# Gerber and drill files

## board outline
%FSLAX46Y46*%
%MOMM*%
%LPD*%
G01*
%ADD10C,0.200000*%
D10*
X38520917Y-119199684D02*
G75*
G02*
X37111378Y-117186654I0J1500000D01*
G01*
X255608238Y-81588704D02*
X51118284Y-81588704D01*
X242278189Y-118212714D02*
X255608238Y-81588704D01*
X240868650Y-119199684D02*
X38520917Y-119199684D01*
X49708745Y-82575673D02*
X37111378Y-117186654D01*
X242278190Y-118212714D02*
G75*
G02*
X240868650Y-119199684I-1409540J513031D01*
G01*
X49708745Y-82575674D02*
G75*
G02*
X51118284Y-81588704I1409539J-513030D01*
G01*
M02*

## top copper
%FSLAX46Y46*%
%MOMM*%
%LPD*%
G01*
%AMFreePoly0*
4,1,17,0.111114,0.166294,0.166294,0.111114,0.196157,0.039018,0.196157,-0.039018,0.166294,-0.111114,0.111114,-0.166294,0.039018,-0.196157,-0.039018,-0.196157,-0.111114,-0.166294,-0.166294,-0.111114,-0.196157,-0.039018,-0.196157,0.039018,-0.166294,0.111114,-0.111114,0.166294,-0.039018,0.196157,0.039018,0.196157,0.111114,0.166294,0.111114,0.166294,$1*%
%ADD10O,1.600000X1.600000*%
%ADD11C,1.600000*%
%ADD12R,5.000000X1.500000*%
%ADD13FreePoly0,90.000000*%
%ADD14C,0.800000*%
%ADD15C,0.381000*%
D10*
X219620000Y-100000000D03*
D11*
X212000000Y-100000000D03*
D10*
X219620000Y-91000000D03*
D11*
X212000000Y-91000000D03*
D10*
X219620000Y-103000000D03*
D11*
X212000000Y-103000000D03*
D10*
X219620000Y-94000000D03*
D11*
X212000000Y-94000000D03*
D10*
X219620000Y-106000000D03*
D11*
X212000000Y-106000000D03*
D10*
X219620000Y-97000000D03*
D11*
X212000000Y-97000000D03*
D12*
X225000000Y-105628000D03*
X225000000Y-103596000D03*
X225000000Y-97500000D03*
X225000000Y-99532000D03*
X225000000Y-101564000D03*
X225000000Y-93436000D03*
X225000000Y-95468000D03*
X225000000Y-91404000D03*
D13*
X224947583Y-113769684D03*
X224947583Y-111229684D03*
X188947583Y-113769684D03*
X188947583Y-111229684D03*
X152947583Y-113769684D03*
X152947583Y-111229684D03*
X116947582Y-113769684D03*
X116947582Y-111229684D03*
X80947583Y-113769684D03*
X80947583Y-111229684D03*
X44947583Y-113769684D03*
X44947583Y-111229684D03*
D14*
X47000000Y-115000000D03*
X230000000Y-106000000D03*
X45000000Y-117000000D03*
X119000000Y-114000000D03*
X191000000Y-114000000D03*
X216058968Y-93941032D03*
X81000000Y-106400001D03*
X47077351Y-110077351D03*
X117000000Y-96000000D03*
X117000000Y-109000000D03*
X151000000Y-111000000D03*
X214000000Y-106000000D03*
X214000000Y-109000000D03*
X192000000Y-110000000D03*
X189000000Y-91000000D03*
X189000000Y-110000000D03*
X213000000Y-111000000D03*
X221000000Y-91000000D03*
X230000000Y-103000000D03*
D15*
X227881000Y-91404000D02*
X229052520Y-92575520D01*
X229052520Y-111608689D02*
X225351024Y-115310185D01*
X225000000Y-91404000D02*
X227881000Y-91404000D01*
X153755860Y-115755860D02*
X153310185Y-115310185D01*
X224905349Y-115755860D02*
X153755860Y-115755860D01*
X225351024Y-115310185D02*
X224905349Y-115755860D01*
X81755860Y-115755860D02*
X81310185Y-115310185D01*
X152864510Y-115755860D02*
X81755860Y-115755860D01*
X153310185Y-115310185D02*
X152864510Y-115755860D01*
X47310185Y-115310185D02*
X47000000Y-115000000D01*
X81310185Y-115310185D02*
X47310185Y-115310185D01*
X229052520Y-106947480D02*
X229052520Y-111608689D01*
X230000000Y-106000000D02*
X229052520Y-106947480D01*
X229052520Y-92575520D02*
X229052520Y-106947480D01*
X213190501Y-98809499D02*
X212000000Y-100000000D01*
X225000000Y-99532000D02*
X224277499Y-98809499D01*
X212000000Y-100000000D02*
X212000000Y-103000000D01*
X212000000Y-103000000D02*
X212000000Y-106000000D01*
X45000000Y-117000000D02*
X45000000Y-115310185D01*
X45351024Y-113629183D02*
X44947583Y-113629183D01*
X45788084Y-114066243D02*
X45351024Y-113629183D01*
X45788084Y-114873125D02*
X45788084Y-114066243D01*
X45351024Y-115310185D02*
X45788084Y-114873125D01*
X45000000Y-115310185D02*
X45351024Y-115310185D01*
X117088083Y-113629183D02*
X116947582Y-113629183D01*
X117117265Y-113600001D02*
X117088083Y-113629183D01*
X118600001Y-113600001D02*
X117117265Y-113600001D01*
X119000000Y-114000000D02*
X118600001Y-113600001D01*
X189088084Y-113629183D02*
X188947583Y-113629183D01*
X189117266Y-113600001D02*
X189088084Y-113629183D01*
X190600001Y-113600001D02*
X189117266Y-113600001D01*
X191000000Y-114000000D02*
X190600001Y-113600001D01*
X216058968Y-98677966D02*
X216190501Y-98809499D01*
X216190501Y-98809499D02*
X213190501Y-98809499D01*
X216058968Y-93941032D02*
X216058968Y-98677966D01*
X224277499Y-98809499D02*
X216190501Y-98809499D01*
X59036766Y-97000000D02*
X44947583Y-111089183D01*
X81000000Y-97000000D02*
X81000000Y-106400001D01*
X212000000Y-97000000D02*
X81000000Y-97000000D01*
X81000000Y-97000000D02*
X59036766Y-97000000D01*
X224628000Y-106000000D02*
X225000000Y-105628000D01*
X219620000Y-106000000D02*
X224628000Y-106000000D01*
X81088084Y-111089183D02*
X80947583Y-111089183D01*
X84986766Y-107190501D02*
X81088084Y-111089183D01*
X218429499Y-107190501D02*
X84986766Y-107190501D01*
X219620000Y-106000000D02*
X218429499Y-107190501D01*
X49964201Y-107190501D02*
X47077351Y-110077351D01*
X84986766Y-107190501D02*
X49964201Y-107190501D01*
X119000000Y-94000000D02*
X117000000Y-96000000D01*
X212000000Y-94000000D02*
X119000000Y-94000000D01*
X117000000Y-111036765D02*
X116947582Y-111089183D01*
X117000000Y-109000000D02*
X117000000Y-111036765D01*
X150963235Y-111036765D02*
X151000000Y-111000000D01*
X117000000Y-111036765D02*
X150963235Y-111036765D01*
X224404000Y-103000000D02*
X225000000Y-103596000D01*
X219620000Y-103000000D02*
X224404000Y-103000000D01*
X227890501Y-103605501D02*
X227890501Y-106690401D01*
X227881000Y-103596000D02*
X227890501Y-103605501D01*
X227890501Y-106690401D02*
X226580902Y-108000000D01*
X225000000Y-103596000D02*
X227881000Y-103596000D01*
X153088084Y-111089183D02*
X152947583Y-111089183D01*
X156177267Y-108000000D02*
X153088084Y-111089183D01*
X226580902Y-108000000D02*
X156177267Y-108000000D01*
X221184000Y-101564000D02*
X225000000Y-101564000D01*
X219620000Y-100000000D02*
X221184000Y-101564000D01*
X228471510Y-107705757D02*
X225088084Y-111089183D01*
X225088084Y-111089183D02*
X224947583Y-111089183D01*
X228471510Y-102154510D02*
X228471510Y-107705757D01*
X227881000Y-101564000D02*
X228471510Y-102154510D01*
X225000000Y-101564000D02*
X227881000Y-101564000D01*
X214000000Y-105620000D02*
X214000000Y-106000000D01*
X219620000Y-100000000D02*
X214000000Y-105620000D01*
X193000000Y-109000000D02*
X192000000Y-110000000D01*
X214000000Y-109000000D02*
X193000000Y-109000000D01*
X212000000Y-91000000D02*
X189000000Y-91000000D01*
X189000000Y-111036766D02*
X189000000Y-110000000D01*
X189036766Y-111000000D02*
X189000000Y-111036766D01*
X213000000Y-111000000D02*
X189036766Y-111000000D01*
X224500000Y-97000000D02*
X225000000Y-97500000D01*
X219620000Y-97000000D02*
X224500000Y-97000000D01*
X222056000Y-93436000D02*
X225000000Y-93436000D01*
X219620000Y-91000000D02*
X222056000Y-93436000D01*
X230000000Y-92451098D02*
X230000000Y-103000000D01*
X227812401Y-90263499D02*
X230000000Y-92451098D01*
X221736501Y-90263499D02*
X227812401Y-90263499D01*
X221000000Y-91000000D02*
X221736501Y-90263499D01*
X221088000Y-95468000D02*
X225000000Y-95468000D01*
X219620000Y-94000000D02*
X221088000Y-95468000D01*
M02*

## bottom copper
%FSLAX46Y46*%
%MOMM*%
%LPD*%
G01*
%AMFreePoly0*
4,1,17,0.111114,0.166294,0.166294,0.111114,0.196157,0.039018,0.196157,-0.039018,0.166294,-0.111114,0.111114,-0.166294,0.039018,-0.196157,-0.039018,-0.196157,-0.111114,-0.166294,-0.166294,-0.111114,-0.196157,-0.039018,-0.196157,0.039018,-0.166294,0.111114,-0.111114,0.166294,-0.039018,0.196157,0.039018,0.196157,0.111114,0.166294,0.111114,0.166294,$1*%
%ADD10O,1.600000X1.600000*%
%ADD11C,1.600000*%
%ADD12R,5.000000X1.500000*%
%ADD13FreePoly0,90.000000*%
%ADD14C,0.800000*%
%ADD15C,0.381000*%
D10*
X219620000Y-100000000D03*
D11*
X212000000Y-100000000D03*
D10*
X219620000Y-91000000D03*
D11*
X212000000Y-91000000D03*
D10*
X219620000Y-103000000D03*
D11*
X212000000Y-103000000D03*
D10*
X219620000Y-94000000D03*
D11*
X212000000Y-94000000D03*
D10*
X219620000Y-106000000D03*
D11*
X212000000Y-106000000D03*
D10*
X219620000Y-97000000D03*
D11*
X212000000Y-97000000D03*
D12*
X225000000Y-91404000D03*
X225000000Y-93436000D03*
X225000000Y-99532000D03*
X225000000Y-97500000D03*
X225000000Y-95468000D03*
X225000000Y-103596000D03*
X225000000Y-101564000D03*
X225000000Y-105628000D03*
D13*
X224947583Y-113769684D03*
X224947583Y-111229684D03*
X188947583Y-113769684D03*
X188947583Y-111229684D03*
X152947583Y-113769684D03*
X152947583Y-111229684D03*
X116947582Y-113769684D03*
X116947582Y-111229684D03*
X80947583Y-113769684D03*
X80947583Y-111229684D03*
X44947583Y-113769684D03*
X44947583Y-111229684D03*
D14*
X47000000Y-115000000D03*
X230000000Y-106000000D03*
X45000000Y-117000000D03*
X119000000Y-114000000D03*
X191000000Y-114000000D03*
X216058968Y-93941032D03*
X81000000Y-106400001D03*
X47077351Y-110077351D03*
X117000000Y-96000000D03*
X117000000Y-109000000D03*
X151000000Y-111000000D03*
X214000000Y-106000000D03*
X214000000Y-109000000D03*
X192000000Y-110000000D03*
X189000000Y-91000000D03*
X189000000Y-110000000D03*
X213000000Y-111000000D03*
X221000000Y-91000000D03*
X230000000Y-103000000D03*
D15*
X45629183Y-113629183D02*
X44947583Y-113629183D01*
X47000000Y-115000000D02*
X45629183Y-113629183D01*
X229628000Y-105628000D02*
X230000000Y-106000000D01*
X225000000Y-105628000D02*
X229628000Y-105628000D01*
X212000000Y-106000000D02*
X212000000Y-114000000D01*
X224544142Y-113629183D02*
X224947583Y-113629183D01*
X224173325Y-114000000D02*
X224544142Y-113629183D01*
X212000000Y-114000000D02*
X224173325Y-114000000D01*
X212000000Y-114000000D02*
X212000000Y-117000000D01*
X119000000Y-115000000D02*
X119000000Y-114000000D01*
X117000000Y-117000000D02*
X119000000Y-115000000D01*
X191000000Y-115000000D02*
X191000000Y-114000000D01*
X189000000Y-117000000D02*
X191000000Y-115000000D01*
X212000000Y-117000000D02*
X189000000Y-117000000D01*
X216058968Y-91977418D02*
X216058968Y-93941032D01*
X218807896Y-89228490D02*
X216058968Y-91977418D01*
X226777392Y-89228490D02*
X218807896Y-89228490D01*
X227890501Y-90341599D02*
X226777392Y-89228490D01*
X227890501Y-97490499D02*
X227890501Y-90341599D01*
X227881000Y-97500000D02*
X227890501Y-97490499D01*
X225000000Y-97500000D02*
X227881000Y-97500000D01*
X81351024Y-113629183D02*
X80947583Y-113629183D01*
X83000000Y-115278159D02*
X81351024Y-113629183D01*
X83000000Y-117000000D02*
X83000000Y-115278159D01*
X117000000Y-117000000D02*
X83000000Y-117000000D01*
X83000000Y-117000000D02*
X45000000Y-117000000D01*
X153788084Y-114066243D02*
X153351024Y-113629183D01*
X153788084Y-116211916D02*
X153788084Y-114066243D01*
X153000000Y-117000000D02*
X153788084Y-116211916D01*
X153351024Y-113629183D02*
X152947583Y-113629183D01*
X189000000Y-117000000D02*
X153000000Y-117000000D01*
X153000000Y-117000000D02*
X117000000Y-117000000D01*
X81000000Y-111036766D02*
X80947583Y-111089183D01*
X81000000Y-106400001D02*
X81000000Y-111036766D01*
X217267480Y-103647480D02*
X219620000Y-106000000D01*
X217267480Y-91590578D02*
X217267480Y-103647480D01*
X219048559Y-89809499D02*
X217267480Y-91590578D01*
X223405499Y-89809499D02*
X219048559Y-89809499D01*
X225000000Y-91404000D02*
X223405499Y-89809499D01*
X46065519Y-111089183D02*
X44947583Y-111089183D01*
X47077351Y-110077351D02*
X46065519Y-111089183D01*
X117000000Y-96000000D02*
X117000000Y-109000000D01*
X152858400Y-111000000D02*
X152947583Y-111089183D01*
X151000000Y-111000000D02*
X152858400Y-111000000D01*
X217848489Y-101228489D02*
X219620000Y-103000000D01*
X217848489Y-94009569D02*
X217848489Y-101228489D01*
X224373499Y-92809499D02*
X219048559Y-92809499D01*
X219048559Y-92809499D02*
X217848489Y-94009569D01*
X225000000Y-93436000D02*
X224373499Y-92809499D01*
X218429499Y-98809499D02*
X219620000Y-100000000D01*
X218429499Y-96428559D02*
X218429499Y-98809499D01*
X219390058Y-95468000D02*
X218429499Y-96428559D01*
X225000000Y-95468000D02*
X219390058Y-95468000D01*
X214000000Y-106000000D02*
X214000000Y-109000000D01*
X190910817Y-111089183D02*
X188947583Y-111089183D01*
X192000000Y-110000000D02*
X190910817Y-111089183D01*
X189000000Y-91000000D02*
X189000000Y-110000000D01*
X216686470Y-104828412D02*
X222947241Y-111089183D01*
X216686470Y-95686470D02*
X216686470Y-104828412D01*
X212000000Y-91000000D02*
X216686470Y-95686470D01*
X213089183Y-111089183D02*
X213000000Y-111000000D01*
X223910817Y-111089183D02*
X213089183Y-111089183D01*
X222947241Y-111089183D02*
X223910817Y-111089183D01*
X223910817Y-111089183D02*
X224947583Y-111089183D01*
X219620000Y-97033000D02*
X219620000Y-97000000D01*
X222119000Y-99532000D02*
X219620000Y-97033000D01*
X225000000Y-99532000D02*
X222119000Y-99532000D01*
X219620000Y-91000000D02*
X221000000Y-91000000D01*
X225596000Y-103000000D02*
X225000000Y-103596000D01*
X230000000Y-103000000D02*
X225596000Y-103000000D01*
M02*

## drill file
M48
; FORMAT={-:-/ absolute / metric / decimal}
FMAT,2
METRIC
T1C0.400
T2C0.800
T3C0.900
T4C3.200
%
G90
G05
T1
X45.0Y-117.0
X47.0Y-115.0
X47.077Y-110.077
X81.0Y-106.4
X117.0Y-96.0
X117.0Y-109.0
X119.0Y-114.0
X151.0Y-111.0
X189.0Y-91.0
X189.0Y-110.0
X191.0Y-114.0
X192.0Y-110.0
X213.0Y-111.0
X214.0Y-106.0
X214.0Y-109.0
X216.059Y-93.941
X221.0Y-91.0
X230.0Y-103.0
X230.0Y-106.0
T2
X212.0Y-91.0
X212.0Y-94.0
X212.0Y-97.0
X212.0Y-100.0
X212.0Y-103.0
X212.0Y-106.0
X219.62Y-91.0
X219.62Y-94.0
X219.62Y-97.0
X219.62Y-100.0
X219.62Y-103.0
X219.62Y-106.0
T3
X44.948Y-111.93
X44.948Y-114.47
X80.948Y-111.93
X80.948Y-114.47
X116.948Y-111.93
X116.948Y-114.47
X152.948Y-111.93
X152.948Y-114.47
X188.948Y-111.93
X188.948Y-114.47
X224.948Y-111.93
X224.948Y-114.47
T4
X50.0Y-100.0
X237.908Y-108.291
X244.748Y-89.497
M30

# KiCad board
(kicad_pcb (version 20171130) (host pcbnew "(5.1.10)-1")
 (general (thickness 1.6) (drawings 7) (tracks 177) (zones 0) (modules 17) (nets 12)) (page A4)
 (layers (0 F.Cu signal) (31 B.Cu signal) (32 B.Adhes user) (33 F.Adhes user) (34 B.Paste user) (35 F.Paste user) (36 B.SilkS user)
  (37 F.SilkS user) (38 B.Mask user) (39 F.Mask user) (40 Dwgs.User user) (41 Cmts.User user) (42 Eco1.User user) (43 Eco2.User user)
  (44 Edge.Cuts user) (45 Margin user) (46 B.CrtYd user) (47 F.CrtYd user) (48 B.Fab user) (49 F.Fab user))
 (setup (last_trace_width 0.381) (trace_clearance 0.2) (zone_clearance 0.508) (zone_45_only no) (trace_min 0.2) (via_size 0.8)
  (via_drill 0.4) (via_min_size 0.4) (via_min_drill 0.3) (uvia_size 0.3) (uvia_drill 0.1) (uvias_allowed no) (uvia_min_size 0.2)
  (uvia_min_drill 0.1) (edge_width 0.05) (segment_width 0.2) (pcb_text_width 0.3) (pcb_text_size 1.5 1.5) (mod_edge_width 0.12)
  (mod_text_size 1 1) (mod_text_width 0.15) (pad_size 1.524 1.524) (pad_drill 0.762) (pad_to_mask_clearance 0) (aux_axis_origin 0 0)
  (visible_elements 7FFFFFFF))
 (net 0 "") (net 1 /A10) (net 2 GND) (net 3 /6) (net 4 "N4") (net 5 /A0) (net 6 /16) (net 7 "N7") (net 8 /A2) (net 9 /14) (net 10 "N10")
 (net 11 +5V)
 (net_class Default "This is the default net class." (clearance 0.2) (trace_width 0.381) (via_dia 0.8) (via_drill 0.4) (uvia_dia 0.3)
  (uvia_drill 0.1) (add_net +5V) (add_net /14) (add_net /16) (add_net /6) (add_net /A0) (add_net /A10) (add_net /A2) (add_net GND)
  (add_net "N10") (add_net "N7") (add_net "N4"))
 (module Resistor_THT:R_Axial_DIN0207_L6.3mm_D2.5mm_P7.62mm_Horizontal (layer F.Cu) (at 212 100)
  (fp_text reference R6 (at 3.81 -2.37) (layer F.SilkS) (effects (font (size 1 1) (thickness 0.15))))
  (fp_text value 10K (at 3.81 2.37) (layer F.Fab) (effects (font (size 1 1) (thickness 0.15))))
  (pad 2 thru_hole oval (at 7.62 0) (size 1.6 1.6) (drill 0.8) (layers *.Cu *.Mask) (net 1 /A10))
  (pad 1 thru_hole circle (at 0 0) (size 1.6 1.6) (drill 0.8) (layers *.Cu *.Mask) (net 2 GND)))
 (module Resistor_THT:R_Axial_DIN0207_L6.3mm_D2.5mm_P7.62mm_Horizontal (layer F.Cu) (at 212 91)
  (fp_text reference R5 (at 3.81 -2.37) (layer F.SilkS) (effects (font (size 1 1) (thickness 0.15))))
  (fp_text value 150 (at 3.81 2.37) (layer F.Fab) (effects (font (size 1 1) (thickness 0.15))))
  (pad 2 thru_hole oval (at 7.62 0) (size 1.6 1.6) (drill 0.8) (layers *.Cu *.Mask) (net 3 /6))
  (pad 1 thru_hole circle (at 0 0) (size 1.6 1.6) (drill 0.8) (layers *.Cu *.Mask) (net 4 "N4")))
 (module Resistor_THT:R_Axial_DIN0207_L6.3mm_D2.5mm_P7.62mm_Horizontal (layer F.Cu) (at 212 103)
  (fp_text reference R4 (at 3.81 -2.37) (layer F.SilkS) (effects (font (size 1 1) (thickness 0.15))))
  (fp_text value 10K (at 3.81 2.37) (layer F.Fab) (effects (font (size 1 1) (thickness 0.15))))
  (pad 2 thru_hole oval (at 7.62 0) (size 1.6 1.6) (drill 0.8) (layers *.Cu *.Mask) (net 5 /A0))
  (pad 1 thru_hole circle (at 0 0) (size 1.6 1.6) (drill 0.8) (layers *.Cu *.Mask) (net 2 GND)))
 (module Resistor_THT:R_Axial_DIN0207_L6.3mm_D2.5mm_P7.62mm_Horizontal (layer F.Cu) (at 212 94)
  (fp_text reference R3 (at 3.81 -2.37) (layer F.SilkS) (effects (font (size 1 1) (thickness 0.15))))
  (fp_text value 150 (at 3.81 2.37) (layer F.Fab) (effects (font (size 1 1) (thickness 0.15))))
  (pad 2 thru_hole oval (at 7.62 0) (size 1.6 1.6) (drill 0.8) (layers *.Cu *.Mask) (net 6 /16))
  (pad 1 thru_hole circle (at 0 0) (size 1.6 1.6) (drill 0.8) (layers *.Cu *.Mask) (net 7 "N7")))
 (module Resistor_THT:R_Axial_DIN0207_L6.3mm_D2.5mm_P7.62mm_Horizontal (layer F.Cu) (at 212 106)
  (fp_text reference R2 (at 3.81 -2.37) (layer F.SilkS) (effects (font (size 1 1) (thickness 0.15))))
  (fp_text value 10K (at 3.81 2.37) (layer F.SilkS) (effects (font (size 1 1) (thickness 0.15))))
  (pad 2 thru_hole oval (at 7.62 0) (size 1.6 1.6) (drill 0.8) (layers *.Cu *.Mask) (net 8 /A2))
  (pad 1 thru_hole circle (at 0 0) (size 1.6 1.6) (drill 0.8) (layers *.Cu *.Mask) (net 2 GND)))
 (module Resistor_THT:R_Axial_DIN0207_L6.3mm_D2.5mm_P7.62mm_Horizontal (layer F.Cu) (at 212 97)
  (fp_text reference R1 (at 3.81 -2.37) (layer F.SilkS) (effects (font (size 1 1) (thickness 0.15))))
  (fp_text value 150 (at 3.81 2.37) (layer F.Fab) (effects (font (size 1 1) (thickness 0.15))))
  (pad 2 thru_hole oval (at 7.62 0) (size 1.6 1.6) (drill 0.8) (layers *.Cu *.Mask) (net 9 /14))
  (pad 1 thru_hole circle (at 0 0) (size 1.6 1.6) (drill 0.8) (layers *.Cu *.Mask) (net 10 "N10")))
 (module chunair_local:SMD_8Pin (layer B.Cu) (at 225 99.532)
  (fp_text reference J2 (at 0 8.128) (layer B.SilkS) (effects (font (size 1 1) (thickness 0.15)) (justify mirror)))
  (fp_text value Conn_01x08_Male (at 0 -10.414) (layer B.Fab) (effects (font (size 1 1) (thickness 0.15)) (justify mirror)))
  (pad 8 smd rect (at 0 -8.128) (size 5 1.5) (layers B.Cu B.Paste B.Mask) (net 8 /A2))
  (pad 7 smd rect (at 0 -6.096) (size 5 1.5) (layers B.Cu B.Paste B.Mask) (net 5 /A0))
  (pad 4 smd rect (at 0 0) (size 5 1.5) (layers B.Cu B.Paste B.Mask) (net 9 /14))
  (pad 5 smd rect (at 0 -2.032) (size 5 1.5) (layers B.Cu B.Paste B.Mask) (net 2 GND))
  (pad 6 smd rect (at 0 -4.064) (size 5 1.5) (layers B.Cu B.Paste B.Mask) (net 1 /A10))
  (pad 2 smd rect (at 0 4.064) (size 5 1.5) (layers B.Cu B.Paste B.Mask) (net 3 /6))
  (pad 3 smd rect (at 0 2.032) (size 5 1.5) (layers B.Cu B.Paste B.Mask) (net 6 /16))
  (pad 1 smd rect (at 0 6.096) (size 5 1.5) (layers B.Cu B.Paste B.Mask) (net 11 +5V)))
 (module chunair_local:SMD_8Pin (layer F.Cu) (at 225 97.5)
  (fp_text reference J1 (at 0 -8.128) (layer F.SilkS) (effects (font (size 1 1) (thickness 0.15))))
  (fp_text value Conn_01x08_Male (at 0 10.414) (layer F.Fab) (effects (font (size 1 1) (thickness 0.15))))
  (pad 8 smd rect (at 0 8.128) (size 5 1.5) (layers F.Cu F.Paste F.Mask) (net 8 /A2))
  (pad 7 smd rect (at 0 6.096) (size 5 1.5) (layers F.Cu F.Paste F.Mask) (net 5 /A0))
  (pad 4 smd rect (at 0 0) (size 5 1.5) (layers F.Cu F.Paste F.Mask) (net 9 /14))
  (pad 5 smd rect (at 0 2.032) (size 5 1.5) (layers F.Cu F.Paste F.Mask) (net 2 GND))
  (pad 6 smd rect (at 0 4.064) (size 5 1.5) (layers F.Cu F.Paste F.Mask) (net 1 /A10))
  (pad 2 smd rect (at 0 -4.064) (size 5 1.5) (layers F.Cu F.Paste F.Mask) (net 3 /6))
  (pad 3 smd rect (at 0 -2.032) (size 5 1.5) (layers F.Cu F.Paste F.Mask) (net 6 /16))
  (pad 1 smd rect (at 0 -6.096) (size 5 1.5) (layers F.Cu F.Paste F.Mask) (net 11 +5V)))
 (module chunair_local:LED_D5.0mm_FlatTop (layer F.Cu) (at 224.947583 114.469684 90)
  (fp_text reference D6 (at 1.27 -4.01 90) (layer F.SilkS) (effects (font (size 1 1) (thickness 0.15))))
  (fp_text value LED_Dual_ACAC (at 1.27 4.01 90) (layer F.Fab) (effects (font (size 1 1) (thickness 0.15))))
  (pad 2 smd custom (at 0.7 0 90) (size 0.4 0.4) (layers F.Cu F.Mask) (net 11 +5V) (zone_connect 0)
   (options (clearance outline) (anchor circle)) (primitives))
  (pad 4 smd custom (at 0.7 0 90) (size 0.4 0.4) (layers B.Cu B.Mask) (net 2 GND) (zone_connect 0)
   (options (clearance outline) (anchor circle)) (primitives))
  (pad 1 smd custom (at 3.24 0 90) (size 0.4 0.4) (layers F.Cu F.Mask) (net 1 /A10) (options (clearance outline) (anchor circle))
   (primitives))
  (pad 3 smd custom (at 3.24 0 90) (size 0.4 0.4) (layers B.Cu B.Mask) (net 4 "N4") (zone_connect 0)
   (options (clearance outline) (anchor circle)) (primitives))
  (pad "" np_thru_hole circle (at 2.54 0 90) (size 0.9 0.9) (drill 0.9) (layers *.Cu *.Mask))
  (pad "" np_thru_hole circle (at 0 0 90) (size 0.9 0.9) (drill 0.9) (layers *.Cu *.Mask)))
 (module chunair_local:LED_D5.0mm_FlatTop (layer F.Cu) (at 188.947583 114.469684 90)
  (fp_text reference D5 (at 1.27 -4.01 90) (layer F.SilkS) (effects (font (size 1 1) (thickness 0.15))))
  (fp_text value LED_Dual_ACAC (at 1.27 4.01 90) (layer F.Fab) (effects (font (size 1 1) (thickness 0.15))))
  (pad 2 smd custom (at 0.7 0 90) (size 0.4 0.4) (layers F.Cu F.Mask) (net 2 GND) (zone_connect 0)
   (options (clearance outline) (anchor circle)) (primitives))
  (pad 4 smd custom (at 0.7 0 90) (size 0.4 0.4) (layers B.Cu B.Mask) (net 11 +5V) (zone_connect 0)
   (options (clearance outline) (anchor circle)) (primitives))
  (pad 1 smd custom (at 3.24 0 90) (size 0.4 0.4) (layers F.Cu F.Mask) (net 4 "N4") (options (clearance outline) (anchor circle))
   (primitives))
  (pad 3 smd custom (at 3.24 0 90) (size 0.4 0.4) (layers B.Cu B.Mask) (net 1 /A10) (zone_connect 0)
   (options (clearance outline) (anchor circle)) (primitives))
  (pad "" np_thru_hole circle (at 2.54 0 90) (size 0.9 0.9) (drill 0.9) (layers *.Cu *.Mask))
  (pad "" np_thru_hole circle (at 0 0 90) (size 0.9 0.9) (drill 0.9) (layers *.Cu *.Mask)))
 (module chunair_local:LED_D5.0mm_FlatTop (layer F.Cu) (at 152.947583 114.469684 90)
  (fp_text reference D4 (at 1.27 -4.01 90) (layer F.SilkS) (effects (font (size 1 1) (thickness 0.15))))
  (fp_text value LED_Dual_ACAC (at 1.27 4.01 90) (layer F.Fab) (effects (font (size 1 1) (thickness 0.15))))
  (pad 2 smd custom (at 0.7 0 90) (size 0.4 0.4) (layers F.Cu F.Mask) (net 11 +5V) (zone_connect 0)
   (options (clearance outline) (anchor circle)) (primitives))
  (pad 4 smd custom (at 0.7 0 90) (size 0.4 0.4) (layers B.Cu B.Mask) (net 2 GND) (zone_connect 0)
   (options (clearance outline) (anchor circle)) (primitives))
  (pad 1 smd custom (at 3.24 0 90) (size 0.4 0.4) (layers F.Cu F.Mask) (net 5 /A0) (options (clearance outline) (anchor circle))
   (primitives))
  (pad 3 smd custom (at 3.24 0 90) (size 0.4 0.4) (layers B.Cu B.Mask) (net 7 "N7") (zone_connect 0)
   (options (clearance outline) (anchor circle)) (primitives))
  (pad "" np_thru_hole circle (at 2.54 0 90) (size 0.9 0.9) (drill 0.9) (layers *.Cu *.Mask))
  (pad "" np_thru_hole circle (at 0 0 90) (size 0.9 0.9) (drill 0.9) (layers *.Cu *.Mask)))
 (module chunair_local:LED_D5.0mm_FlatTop (layer F.Cu) (at 116.947582 114.469684 90)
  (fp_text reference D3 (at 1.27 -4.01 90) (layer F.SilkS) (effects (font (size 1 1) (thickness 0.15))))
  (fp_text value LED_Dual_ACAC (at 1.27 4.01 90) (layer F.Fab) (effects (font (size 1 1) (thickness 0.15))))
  (pad 2 smd custom (at 0.7 0 90) (size 0.4 0.4) (layers F.Cu F.Mask) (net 2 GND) (zone_connect 0)
   (options (clearance outline) (anchor circle)) (primitives))
  (pad 4 smd custom (at 0.7 0 90) (size 0.4 0.4) (layers B.Cu B.Mask) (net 11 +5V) (zone_connect 0)
   (options (clearance outline) (anchor circle)) (primitives))
  (pad 1 smd custom (at 3.24 0 90) (size 0.4 0.4) (layers F.Cu F.Mask) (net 7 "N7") (options (clearance outline) (anchor circle))
   (primitives))
  (pad 3 smd custom (at 3.24 0 90) (size 0.4 0.4) (layers B.Cu B.Mask) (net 5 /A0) (zone_connect 0)
   (options (clearance outline) (anchor circle)) (primitives))
  (pad "" np_thru_hole circle (at 2.54 0 90) (size 0.9 0.9) (drill 0.9) (layers *.Cu *.Mask))
  (pad "" np_thru_hole circle (at 0 0 90) (size 0.9 0.9) (drill 0.9) (layers *.Cu *.Mask)))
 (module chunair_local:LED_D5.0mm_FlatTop (layer F.Cu) (at 80.947583 114.469684 90)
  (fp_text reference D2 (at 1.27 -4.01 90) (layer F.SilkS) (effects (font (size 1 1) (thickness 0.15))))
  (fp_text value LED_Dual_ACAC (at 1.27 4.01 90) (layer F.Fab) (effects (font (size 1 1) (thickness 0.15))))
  (pad 2 smd custom (at 0.7 0 90) (size 0.4 0.4) (layers F.Cu F.Mask) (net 11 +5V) (zone_connect 0)
   (options (clearance outline) (anchor circle)) (primitives))
  (pad 4 smd custom (at 0.7 0 90) (size 0.4 0.4) (layers B.Cu B.Mask) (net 2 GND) (zone_connect 0)
   (options (clearance outline) (anchor circle)) (primitives))
  (pad 1 smd custom (at 3.24 0 90) (size 0.4 0.4) (layers F.Cu F.Mask) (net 8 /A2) (options (clearance outline) (anchor circle))
   (primitives))
  (pad 3 smd custom (at 3.24 0 90) (size 0.4 0.4) (layers B.Cu B.Mask) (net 10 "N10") (zone_connect 0)
   (options (clearance outline) (anchor circle)) (primitives))
  (pad "" np_thru_hole circle (at 2.54 0 90) (size 0.9 0.9) (drill 0.9) (layers *.Cu *.Mask))
  (pad "" np_thru_hole circle (at 0 0 90) (size 0.9 0.9) (drill 0.9) (layers *.Cu *.Mask)))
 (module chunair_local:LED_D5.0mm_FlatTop (layer F.Cu) (at 44.947583 114.469684 90)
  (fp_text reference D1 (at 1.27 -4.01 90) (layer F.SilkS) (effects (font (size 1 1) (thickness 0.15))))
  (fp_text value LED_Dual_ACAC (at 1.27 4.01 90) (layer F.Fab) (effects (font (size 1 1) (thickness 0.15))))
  (pad 2 smd custom (at 0.7 0 90) (size 0.4 0.4) (layers F.Cu F.Mask) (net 2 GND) (zone_connect 0)
   (options (clearance outline) (anchor circle)) (primitives))
  (pad 4 smd custom (at 0.7 0 90) (size 0.4 0.4) (layers B.Cu B.Mask) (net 11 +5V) (zone_connect 0)
   (options (clearance outline) (anchor circle)) (primitives))
  (pad 1 smd custom (at 3.24 0 90) (size 0.4 0.4) (layers F.Cu F.Mask) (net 10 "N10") (options (clearance outline) (anchor circle))
   (primitives))
  (pad 3 smd custom (at 3.24 0 90) (size 0.4 0.4) (layers B.Cu B.Mask) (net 8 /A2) (zone_connect 0)
   (options (clearance outline) (anchor circle)) (primitives))
  (pad "" np_thru_hole circle (at 2.54 0 90) (size 0.9 0.9) (drill 0.9) (layers *.Cu *.Mask))
  (pad "" np_thru_hole circle (at 0 0 90) (size 0.9 0.9) (drill 0.9) (layers *.Cu *.Mask)))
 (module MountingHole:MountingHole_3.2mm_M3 (layer F.Cu) (at 244.748423 89.497267)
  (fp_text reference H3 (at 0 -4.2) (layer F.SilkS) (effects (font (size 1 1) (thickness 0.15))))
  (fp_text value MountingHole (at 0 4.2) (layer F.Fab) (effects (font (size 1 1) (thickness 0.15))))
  (pad 1 np_thru_hole circle (at 0 0) (size 3.2 3.2) (drill 3.2) (layers *.Cu *.Mask)))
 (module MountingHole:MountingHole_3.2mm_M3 (layer F.Cu) (at 237.90802 108.29112)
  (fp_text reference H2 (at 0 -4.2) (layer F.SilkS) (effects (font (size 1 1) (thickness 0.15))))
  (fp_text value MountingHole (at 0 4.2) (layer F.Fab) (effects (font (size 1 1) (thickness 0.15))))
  (pad 1 np_thru_hole circle (at 0 0) (size 3.2 3.2) (drill 3.2) (layers *.Cu *.Mask)))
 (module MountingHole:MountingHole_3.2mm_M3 (layer F.Cu) (at 50 100)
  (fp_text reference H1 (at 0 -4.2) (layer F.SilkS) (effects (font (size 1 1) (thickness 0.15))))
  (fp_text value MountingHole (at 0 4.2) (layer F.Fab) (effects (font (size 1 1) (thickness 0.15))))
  (pad 1 np_thru_hole circle (at 0 0) (size 3.2 3.2) (drill 3.2) (layers *.Cu *.Mask)))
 (gr_arc (start 38.520917 117.699684) (end 37.111378 117.186654) (angle -110) (layer Edge.Cuts) (width 0.2))
 (gr_line (start 255.608238 81.588704) (end 51.118284 81.588704) (layer Edge.Cuts) (width 0.2))
 (gr_line (start 242.278189 118.212714) (end 255.608238 81.588704) (layer Edge.Cuts) (width 0.2))
 (gr_line (start 240.86865 119.199684) (end 38.520917 119.199684) (layer Edge.Cuts) (width 0.2))
 (gr_line (start 49.708745 82.575673) (end 37.111378 117.186654) (layer Edge.Cuts) (width 0.2))
 (gr_arc (start 240.86865 117.699683) (end 240.86865 119.199684) (angle -70) (layer Edge.Cuts) (width 0.2))
 (gr_arc (start 51.118284 83.088704) (end 51.118284 81.588704) (angle -70) (layer Edge.Cuts) (width 0.2))
 (segment (start 227.881 91.404) (end 229.05252 92.57552) (width 0.381) (layer F.Cu) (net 11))
 (segment (start 229.05252 111.608689) (end 225.351024 115.310185) (width 0.381) (layer F.Cu) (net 11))
 (segment (start 225 91.404) (end 227.881 91.404) (width 0.381) (layer F.Cu) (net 11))
 (segment (start 153.75586 115.75586) (end 153.310185 115.310185) (width 0.381) (layer F.Cu) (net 11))
 (segment (start 224.905349 115.75586) (end 153.75586 115.75586) (width 0.381) (layer F.Cu) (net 11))
 (segment (start 225.351024 115.310185) (end 224.905349 115.75586) (width 0.381) (layer F.Cu) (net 11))
 (segment (start 81.75586 115.75586) (end 81.310185 115.310185) (width 0.381) (layer F.Cu) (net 11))
 (segment (start 152.86451 115.75586) (end 81.75586 115.75586) (width 0.381) (layer F.Cu) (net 11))
 (segment (start 153.310185 115.310185) (end 152.86451 115.75586) (width 0.381) (layer F.Cu) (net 11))
 (via (at 47 115) (size 0.8) (drill 0.4) (layers F.Cu B.Cu) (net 11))
 (segment (start 47.310185 115.310185) (end 47 115) (width 0.381) (layer F.Cu) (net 11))
 (segment (start 81.310185 115.310185) (end 47.310185 115.310185) (width 0.381) (layer F.Cu) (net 11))
 (segment (start 45.629183 113.629183) (end 44.947583 113.629183) (width 0.381) (layer B.Cu) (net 11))
 (segment (start 47 115) (end 45.629183 113.629183) (width 0.381) (layer B.Cu) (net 11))
 (via (at 230 106) (size 0.8) (drill 0.4) (layers F.Cu B.Cu) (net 11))
 (segment (start 229.628 105.628) (end 230 106) (width 0.381) (layer B.Cu) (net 11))
 (segment (start 225 105.628) (end 229.628 105.628) (width 0.381) (layer B.Cu) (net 11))
 (segment (start 229.05252 106.94748) (end 229.05252 111.608689) (width 0.381) (layer F.Cu) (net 11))
 (segment (start 230 106) (end 229.05252 106.94748) (width 0.381) (layer F.Cu) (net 11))
 (segment (start 229.05252 92.57552) (end 229.05252 106.94748) (width 0.381) (layer F.Cu) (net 11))
 (segment (start 213.190501 98.809499) (end 212 100) (width 0.381) (layer F.Cu) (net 2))
 (segment (start 225 99.532) (end 224.277499 98.809499) (width 0.381) (layer F.Cu) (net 2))
 (segment (start 212 100) (end 212 103) (width 0.381) (layer F.Cu) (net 2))
 (segment (start 212 103) (end 212 106) (width 0.381) (layer F.Cu) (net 2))
 (segment (start 212 106) (end 212 114) (width 0.381) (layer B.Cu) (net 2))
 (segment (start 224.544142 113.629183) (end 224.947583 113.629183) (width 0.381) (layer B.Cu) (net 2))
 (segment (start 224.173325 114) (end 224.544142 113.629183) (width 0.381) (layer B.Cu) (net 2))
 (segment (start 212 114) (end 224.173325 114) (width 0.381) (layer B.Cu) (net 2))
 (segment (start 212 114) (end 212 117) (width 0.381) (layer B.Cu) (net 2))
 (via (at 45 117) (size 0.8) (drill 0.4) (layers F.Cu B.Cu) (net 2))
 (segment (start 45 117) (end 45 115.310185) (width 0.381) (layer F.Cu) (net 2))
 (segment (start 45.351024 113.629183) (end 44.947583 113.629183) (width 0.381) (layer F.Cu) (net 2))
 (segment (start 45.788084 114.066243) (end 45.351024 113.629183) (width 0.381) (layer F.Cu) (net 2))
 (segment (start 45.788084 114.873125) (end 45.788084 114.066243) (width 0.381) (layer F.Cu) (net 2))
 (segment (start 45.351024 115.310185) (end 45.788084 114.873125) (width 0.381) (layer F.Cu) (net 2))
 (segment (start 45 115.310185) (end 45.351024 115.310185) (width 0.381) (layer F.Cu) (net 2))
 (via (at 119 114) (size 0.8) (drill 0.4) (layers F.Cu B.Cu) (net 2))
 (segment (start 119 115) (end 119 114) (width 0.381) (layer B.Cu) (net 2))
 (segment (start 117 117) (end 119 115) (width 0.381) (layer B.Cu) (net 2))
 (segment (start 117.088083 113.629183) (end 116.947582 113.629183) (width 0.381) (layer F.Cu) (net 2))
 (segment (start 117.117265 113.600001) (end 117.088083 113.629183) (width 0.381) (layer F.Cu) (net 2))
 (segment (start 118.600001 113.600001) (end 117.117265 113.600001) (width 0.381) (layer F.Cu) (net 2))
 (segment (start 119 114) (end 118.600001 113.600001) (width 0.381) (layer F.Cu) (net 2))
 (via (at 191 114) (size 0.8) (drill 0.4) (layers F.Cu B.Cu) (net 2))
 (segment (start 191 115) (end 191 114) (width 0.381) (layer B.Cu) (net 2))
 (segment (start 189 117) (end 191 115) (width 0.381) (layer B.Cu) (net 2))
 (segment (start 212 117) (end 189 117) (width 0.381) (layer B.Cu) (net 2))
 (segment (start 189.088084 113.629183) (end 188.947583 113.629183) (width 0.381) (layer F.Cu) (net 2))
 (segment (start 189.117266 113.600001) (end 189.088084 113.629183) (width 0.381) (layer F.Cu) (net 2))
 (segment (start 190.600001 113.600001) (end 189.117266 113.600001) (width 0.381) (layer F.Cu) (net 2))
 (segment (start 191 114) (end 190.600001 113.600001) (width 0.381) (layer F.Cu) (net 2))
 (segment (start 216.058968 91.977418) (end 216.058968 93.941032) (width 0.381) (layer B.Cu) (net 2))
 (via (at 216.058968 93.941032) (size 0.8) (drill 0.4) (layers F.Cu B.Cu) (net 2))
 (segment (start 218.807896 89.22849) (end 216.058968 91.977418) (width 0.381) (layer B.Cu) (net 2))
 (segment (start 226.777392 89.22849) (end 218.807896 89.22849) (width 0.381) (layer B.Cu) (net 2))
 (segment (start 227.890501 90.341599) (end 226.777392 89.22849) (width 0.381) (layer B.Cu) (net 2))
 (segment (start 227.890501 97.490499) (end 227.890501 90.341599) (width 0.381) (layer B.Cu) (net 2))
 (segment (start 227.881 97.5) (end 227.890501 97.490499) (width 0.381) (layer B.Cu) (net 2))
 (segment (start 225 97.5) (end 227.881 97.5) (width 0.381) (layer B.Cu) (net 2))
 (segment (start 216.058968 98.677966) (end 216.190501 98.809499) (width 0.381) (layer F.Cu) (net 2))
 (segment (start 216.190501 98.809499) (end 213.190501 98.809499) (width 0.381) (layer F.Cu) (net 2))
 (segment (start 216.058968 93.941032) (end 216.058968 98.677966) (width 0.381) (layer F.Cu) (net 2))
 (segment (start 224.277499 98.809499) (end 216.190501 98.809499) (width 0.381) (layer F.Cu) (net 2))
 (segment (start 81.351024 113.629183) (end 80.947583 113.629183) (width 0.381) (layer B.Cu) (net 2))
 (segment (start 83 115.278159) (end 81.351024 113.629183) (width 0.381) (layer B.Cu) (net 2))
 (segment (start 83 117) (end 83 115.278159) (width 0.381) (layer B.Cu) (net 2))
 (segment (start 117 117) (end 83 117) (width 0.381) (layer B.Cu) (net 2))
 (segment (start 83 117) (end 45 117) (width 0.381) (layer B.Cu) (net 2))
 (segment (start 153.788084 114.066243) (end 153.351024 113.629183) (width 0.381) (layer B.Cu) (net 2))
 (segment (start 153.788084 116.211916) (end 153.788084 114.066243) (width 0.381) (layer B.Cu) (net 2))
 (segment (start 153 117) (end 153.788084 116.211916) (width 0.381) (layer B.Cu) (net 2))
 (segment (start 153.351024 113.629183) (end 152.947583 113.629183) (width 0.381) (layer B.Cu) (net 2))
 (segment (start 189 117) (end 153 117) (width 0.381) (layer B.Cu) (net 2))
 (segment (start 153 117) (end 117 117) (width 0.381) (layer B.Cu) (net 2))
 (segment (start 59.036766 97) (end 44.947583 111.089183) (width 0.381) (layer F.Cu) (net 10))
 (segment (start 81 97) (end 81 106.400001) (width 0.381) (layer F.Cu) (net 10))
 (segment (start 212 97) (end 81 97) (width 0.381) (layer F.Cu) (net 10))
 (via (at 81 106.400001) (size 0.8) (drill 0.4) (layers F.Cu B.Cu) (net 10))
 (segment (start 81 97) (end 59.036766 97) (width 0.381) (layer F.Cu) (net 10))
 (segment (start 81 111.036766) (end 80.947583 111.089183) (width 0.381) (layer B.Cu) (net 10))
 (segment (start 81 106.400001) (end 81 111.036766) (width 0.381) (layer B.Cu) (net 10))
 (segment (start 224.628 106) (end 225 105.628) (width 0.381) (layer F.Cu) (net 8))
 (segment (start 219.62 106) (end 224.628 106) (width 0.381) (layer F.Cu) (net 8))
 (segment (start 81.088084 111.089183) (end 80.947583 111.089183) (width 0.381) (layer F.Cu) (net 8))
 (segment (start 84.986766 107.190501) (end 81.088084 111.089183) (width 0.381) (layer F.Cu) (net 8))
 (segment (start 218.429499 107.190501) (end 84.986766 107.190501) (width 0.381) (layer F.Cu) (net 8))
 (segment (start 219.62 106) (end 218.429499 107.190501) (width 0.381) (layer F.Cu) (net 8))
 (segment (start 217.26748 103.64748) (end 219.62 106) (width 0.381) (layer B.Cu) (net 8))
 (segment (start 217.26748 91.590578) (end 217.26748 103.64748) (width 0.381) (layer B.Cu) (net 8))
 (segment (start 219.048559 89.809499) (end 217.26748 91.590578) (width 0.381) (layer B.Cu) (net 8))
 (segment (start 223.405499 89.809499) (end 219.048559 89.809499) (width 0.381) (layer B.Cu) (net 8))
 (segment (start 225 91.404) (end 223.405499 89.809499) (width 0.381) (layer B.Cu) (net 8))
 (via (at 47.077351 110.077351) (size 0.8) (drill 0.4) (layers F.Cu B.Cu) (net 8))
 (segment (start 49.964201 107.190501) (end 47.077351 110.077351) (width 0.381) (layer F.Cu) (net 8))
 (segment (start 84.986766 107.190501) (end 49.964201 107.190501) (width 0.381) (layer F.Cu) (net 8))
 (segment (start 46.065519 111.089183) (end 44.947583 111.089183) (width 0.381) (layer B.Cu) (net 8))
 (segment (start 47.077351 110.077351) (end 46.065519 111.089183) (width 0.381) (layer B.Cu) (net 8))
 (via (at 117 96) (size 0.8) (drill 0.4) (layers F.Cu B.Cu) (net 7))
 (segment (start 119 94) (end 117 96) (width 0.381) (layer F.Cu) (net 7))
 (segment (start 212 94) (end 119 94) (width 0.381) (layer F.Cu) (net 7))
 (via (at 117 109) (size 0.8) (drill 0.4) (layers F.Cu B.Cu) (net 7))
 (segment (start 117 96) (end 117 109) (width 0.381) (layer B.Cu) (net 7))
 (segment (start 117 111.036765) (end 116.947582 111.089183) (width 0.381) (layer F.Cu) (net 7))
 (segment (start 117 109) (end 117 111.036765) (width 0.381) (layer F.Cu) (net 7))
 (via (at 151 111) (size 0.8) (drill 0.4) (layers F.Cu B.Cu) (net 7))
 (segment (start 150.963235 111.036765) (end 151 111) (width 0.381) (layer F.Cu) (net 7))
 (segment (start 117 111.036765) (end 150.963235 111.036765) (width 0.381) (layer F.Cu) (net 7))
 (segment (start 152.8584 111) (end 152.947583 111.089183) (width 0.381) (layer B.Cu) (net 7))
 (segment (start 151 111) (end 152.8584 111) (width 0.381) (layer B.Cu) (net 7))
 (segment (start 224.404 103) (end 225 103.596) (width 0.381) (layer F.Cu) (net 5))
 (segment (start 219.62 103) (end 224.404 103) (width 0.381) (layer F.Cu) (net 5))
 (segment (start 227.890501 103.605501) (end 227.890501 106.690401) (width 0.381) (layer F.Cu) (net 5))
 (segment (start 227.881 103.596) (end 227.890501 103.605501) (width 0.381) (layer F.Cu) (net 5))
 (segment (start 227.890501 106.690401) (end 226.580902 108) (width 0.381) (layer F.Cu) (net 5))
 (segment (start 225 103.596) (end 227.881 103.596) (width 0.381) (layer F.Cu) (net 5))
 (segment (start 153.088084 111.089183) (end 152.947583 111.089183) (width 0.381) (layer F.Cu) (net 5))
 (segment (start 156.177267 108) (end 153.088084 111.089183) (width 0.381) (layer F.Cu) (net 5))
 (segment (start 226.580902 108) (end 156.177267 108) (width 0.381) (layer F.Cu) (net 5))
 (segment (start 217.848489 101.228489) (end 219.62 103) (width 0.381) (layer B.Cu) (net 5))
 (segment (start 217.848489 94.009569) (end 217.848489 101.228489) (width 0.381) (layer B.Cu) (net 5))
 (segment (start 224.373499 92.809499) (end 219.048559 92.809499) (width 0.381) (layer B.Cu) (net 5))
 (segment (start 219.048559 92.809499) (end 217.848489 94.009569) (width 0.381) (layer B.Cu) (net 5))
 (segment (start 225 93.436) (end 224.373499 92.809499) (width 0.381) (layer B.Cu) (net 5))
 (segment (start 221.184 101.564) (end 225 101.564) (width 0.381) (layer F.Cu) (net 1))
 (segment (start 219.62 100) (end 221.184 101.564) (width 0.381) (layer F.Cu) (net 1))
 (segment (start 228.47151 107.705757) (end 225.088084 111.089183) (width 0.381) (layer F.Cu) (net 1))
 (segment (start 225.088084 111.089183) (end 224.947583 111.089183) (width 0.381) (layer F.Cu) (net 1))
 (segment (start 228.47151 102.15451) (end 228.47151 107.705757) (width 0.381) (layer F.Cu) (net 1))
 (segment (start 227.881 101.564) (end 228.47151 102.15451) (width 0.381) (layer F.Cu) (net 1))
 (segment (start 225 101.564) (end 227.881 101.564) (width 0.381) (layer F.Cu) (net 1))
 (segment (start 218.429499 98.809499) (end 219.62 100) (width 0.381) (layer B.Cu) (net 1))
 (segment (start 218.429499 96.428559) (end 218.429499 98.809499) (width 0.381) (layer B.Cu) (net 1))
 (segment (start 219.390058 95.468) (end 218.429499 96.428559) (width 0.381) (layer B.Cu) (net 1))
 (segment (start 225 95.468) (end 219.390058 95.468) (width 0.381) (layer B.Cu) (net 1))
 (via (at 214 106) (size 0.8) (drill 0.4) (layers F.Cu B.Cu) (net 1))
 (segment (start 214 105.62) (end 214 106) (width 0.381) (layer F.Cu) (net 1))
 (segment (start 219.62 100) (end 214 105.62) (width 0.381) (layer F.Cu) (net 1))
 (via (at 214 109) (size 0.8) (drill 0.4) (layers F.Cu B.Cu) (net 1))
 (segment (start 214 106) (end 214 109) (width 0.381) (layer B.Cu) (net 1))
 (via (at 192 110) (size 0.8) (drill 0.4) (layers F.Cu B.Cu) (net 1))
 (segment (start 193 109) (end 192 110) (width 0.381) (layer F.Cu) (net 1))
 (segment (start 214 109) (end 193 109) (width 0.381) (layer F.Cu) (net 1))
 (segment (start 190.910817 111.089183) (end 188.947583 111.089183) (width 0.381) (layer B.Cu) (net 1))
 (segment (start 192 110) (end 190.910817 111.089183) (width 0.381) (layer B.Cu) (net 1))
 (via (at 189 91) (size 0.8) (drill 0.4) (layers F.Cu B.Cu) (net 4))
 (segment (start 212 91) (end 189 91) (width 0.381) (layer F.Cu) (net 4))
 (via (at 189 110) (size 0.8) (drill 0.4) (layers F.Cu B.Cu) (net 4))
 (segment (start 189 91) (end 189 110) (width 0.381) (layer B.Cu) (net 4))
 (segment (start 216.68647 104.828412) (end 222.947241 111.089183) (width 0.381) (layer B.Cu) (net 4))
 (segment (start 216.68647 95.68647) (end 216.68647 104.828412) (width 0.381) (layer B.Cu) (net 4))
 (segment (start 212 91) (end 216.68647 95.68647) (width 0.381) (layer B.Cu) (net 4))
 (via (at 213 111) (size 0.8) (drill 0.4) (layers F.Cu B.Cu) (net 4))
 (segment (start 213.089183 111.089183) (end 213 111) (width 0.381) (layer B.Cu) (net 4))
 (segment (start 223.910817 111.089183) (end 213.089183 111.089183) (width 0.381) (layer B.Cu) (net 4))
 (segment (start 222.947241 111.089183) (end 223.910817 111.089183) (width 0.381) (layer B.Cu) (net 4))
 (segment (start 223.910817 111.089183) (end 224.947583 111.089183) (width 0.381) (layer B.Cu) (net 4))
 (segment (start 189 111.036766) (end 189 110) (width 0.381) (layer F.Cu) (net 4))
 (segment (start 189.036766 111) (end 189 111.036766) (width 0.381) (layer F.Cu) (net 4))
 (segment (start 213 111) (end 189.036766 111) (width 0.381) (layer F.Cu) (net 4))
 (segment (start 224.5 97) (end 225 97.5) (width 0.381) (layer F.Cu) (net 9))
 (segment (start 219.62 97) (end 224.5 97) (width 0.381) (layer F.Cu) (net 9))
 (segment (start 219.62 97.033) (end 219.62 97) (width 0.381) (layer B.Cu) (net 9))
 (segment (start 222.119 99.532) (end 219.62 97.033) (width 0.381) (layer B.Cu) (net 9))
 (segment (start 225 99.532) (end 222.119 99.532) (width 0.381) (layer B.Cu) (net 9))
 (segment (start 222.056 93.436) (end 225 93.436) (width 0.381) (layer F.Cu) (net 3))
 (segment (start 219.62 91) (end 222.056 93.436) (width 0.381) (layer F.Cu) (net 3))
 (via (at 221 91) (size 0.8) (drill 0.4) (layers F.Cu B.Cu) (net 3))
 (segment (start 219.62 91) (end 221 91) (width 0.381) (layer B.Cu) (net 3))
 (via (at 230 103) (size 0.8) (drill 0.4) (layers F.Cu B.Cu) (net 3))
 (segment (start 230 92.451098) (end 230 103) (width 0.381) (layer F.Cu) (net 3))
 (segment (start 227.812401 90.263499) (end 230 92.451098) (width 0.381) (layer F.Cu) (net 3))
 (segment (start 221.736501 90.263499) (end 227.812401 90.263499) (width 0.381) (layer F.Cu) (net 3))
 (segment (start 221 91) (end 221.736501 90.263499) (width 0.381) (layer F.Cu) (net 3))
 (segment (start 225.596 103) (end 225 103.596) (width 0.381) (layer B.Cu) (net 3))
 (segment (start 230 103) (end 225.596 103) (width 0.381) (layer B.Cu) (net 3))
 (segment (start 221.088 95.468) (end 225 95.468) (width 0.381) (layer F.Cu) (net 6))
 (segment (start 219.62 94) (end 221.088 95.468) (width 0.381) (layer F.Cu) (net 6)))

